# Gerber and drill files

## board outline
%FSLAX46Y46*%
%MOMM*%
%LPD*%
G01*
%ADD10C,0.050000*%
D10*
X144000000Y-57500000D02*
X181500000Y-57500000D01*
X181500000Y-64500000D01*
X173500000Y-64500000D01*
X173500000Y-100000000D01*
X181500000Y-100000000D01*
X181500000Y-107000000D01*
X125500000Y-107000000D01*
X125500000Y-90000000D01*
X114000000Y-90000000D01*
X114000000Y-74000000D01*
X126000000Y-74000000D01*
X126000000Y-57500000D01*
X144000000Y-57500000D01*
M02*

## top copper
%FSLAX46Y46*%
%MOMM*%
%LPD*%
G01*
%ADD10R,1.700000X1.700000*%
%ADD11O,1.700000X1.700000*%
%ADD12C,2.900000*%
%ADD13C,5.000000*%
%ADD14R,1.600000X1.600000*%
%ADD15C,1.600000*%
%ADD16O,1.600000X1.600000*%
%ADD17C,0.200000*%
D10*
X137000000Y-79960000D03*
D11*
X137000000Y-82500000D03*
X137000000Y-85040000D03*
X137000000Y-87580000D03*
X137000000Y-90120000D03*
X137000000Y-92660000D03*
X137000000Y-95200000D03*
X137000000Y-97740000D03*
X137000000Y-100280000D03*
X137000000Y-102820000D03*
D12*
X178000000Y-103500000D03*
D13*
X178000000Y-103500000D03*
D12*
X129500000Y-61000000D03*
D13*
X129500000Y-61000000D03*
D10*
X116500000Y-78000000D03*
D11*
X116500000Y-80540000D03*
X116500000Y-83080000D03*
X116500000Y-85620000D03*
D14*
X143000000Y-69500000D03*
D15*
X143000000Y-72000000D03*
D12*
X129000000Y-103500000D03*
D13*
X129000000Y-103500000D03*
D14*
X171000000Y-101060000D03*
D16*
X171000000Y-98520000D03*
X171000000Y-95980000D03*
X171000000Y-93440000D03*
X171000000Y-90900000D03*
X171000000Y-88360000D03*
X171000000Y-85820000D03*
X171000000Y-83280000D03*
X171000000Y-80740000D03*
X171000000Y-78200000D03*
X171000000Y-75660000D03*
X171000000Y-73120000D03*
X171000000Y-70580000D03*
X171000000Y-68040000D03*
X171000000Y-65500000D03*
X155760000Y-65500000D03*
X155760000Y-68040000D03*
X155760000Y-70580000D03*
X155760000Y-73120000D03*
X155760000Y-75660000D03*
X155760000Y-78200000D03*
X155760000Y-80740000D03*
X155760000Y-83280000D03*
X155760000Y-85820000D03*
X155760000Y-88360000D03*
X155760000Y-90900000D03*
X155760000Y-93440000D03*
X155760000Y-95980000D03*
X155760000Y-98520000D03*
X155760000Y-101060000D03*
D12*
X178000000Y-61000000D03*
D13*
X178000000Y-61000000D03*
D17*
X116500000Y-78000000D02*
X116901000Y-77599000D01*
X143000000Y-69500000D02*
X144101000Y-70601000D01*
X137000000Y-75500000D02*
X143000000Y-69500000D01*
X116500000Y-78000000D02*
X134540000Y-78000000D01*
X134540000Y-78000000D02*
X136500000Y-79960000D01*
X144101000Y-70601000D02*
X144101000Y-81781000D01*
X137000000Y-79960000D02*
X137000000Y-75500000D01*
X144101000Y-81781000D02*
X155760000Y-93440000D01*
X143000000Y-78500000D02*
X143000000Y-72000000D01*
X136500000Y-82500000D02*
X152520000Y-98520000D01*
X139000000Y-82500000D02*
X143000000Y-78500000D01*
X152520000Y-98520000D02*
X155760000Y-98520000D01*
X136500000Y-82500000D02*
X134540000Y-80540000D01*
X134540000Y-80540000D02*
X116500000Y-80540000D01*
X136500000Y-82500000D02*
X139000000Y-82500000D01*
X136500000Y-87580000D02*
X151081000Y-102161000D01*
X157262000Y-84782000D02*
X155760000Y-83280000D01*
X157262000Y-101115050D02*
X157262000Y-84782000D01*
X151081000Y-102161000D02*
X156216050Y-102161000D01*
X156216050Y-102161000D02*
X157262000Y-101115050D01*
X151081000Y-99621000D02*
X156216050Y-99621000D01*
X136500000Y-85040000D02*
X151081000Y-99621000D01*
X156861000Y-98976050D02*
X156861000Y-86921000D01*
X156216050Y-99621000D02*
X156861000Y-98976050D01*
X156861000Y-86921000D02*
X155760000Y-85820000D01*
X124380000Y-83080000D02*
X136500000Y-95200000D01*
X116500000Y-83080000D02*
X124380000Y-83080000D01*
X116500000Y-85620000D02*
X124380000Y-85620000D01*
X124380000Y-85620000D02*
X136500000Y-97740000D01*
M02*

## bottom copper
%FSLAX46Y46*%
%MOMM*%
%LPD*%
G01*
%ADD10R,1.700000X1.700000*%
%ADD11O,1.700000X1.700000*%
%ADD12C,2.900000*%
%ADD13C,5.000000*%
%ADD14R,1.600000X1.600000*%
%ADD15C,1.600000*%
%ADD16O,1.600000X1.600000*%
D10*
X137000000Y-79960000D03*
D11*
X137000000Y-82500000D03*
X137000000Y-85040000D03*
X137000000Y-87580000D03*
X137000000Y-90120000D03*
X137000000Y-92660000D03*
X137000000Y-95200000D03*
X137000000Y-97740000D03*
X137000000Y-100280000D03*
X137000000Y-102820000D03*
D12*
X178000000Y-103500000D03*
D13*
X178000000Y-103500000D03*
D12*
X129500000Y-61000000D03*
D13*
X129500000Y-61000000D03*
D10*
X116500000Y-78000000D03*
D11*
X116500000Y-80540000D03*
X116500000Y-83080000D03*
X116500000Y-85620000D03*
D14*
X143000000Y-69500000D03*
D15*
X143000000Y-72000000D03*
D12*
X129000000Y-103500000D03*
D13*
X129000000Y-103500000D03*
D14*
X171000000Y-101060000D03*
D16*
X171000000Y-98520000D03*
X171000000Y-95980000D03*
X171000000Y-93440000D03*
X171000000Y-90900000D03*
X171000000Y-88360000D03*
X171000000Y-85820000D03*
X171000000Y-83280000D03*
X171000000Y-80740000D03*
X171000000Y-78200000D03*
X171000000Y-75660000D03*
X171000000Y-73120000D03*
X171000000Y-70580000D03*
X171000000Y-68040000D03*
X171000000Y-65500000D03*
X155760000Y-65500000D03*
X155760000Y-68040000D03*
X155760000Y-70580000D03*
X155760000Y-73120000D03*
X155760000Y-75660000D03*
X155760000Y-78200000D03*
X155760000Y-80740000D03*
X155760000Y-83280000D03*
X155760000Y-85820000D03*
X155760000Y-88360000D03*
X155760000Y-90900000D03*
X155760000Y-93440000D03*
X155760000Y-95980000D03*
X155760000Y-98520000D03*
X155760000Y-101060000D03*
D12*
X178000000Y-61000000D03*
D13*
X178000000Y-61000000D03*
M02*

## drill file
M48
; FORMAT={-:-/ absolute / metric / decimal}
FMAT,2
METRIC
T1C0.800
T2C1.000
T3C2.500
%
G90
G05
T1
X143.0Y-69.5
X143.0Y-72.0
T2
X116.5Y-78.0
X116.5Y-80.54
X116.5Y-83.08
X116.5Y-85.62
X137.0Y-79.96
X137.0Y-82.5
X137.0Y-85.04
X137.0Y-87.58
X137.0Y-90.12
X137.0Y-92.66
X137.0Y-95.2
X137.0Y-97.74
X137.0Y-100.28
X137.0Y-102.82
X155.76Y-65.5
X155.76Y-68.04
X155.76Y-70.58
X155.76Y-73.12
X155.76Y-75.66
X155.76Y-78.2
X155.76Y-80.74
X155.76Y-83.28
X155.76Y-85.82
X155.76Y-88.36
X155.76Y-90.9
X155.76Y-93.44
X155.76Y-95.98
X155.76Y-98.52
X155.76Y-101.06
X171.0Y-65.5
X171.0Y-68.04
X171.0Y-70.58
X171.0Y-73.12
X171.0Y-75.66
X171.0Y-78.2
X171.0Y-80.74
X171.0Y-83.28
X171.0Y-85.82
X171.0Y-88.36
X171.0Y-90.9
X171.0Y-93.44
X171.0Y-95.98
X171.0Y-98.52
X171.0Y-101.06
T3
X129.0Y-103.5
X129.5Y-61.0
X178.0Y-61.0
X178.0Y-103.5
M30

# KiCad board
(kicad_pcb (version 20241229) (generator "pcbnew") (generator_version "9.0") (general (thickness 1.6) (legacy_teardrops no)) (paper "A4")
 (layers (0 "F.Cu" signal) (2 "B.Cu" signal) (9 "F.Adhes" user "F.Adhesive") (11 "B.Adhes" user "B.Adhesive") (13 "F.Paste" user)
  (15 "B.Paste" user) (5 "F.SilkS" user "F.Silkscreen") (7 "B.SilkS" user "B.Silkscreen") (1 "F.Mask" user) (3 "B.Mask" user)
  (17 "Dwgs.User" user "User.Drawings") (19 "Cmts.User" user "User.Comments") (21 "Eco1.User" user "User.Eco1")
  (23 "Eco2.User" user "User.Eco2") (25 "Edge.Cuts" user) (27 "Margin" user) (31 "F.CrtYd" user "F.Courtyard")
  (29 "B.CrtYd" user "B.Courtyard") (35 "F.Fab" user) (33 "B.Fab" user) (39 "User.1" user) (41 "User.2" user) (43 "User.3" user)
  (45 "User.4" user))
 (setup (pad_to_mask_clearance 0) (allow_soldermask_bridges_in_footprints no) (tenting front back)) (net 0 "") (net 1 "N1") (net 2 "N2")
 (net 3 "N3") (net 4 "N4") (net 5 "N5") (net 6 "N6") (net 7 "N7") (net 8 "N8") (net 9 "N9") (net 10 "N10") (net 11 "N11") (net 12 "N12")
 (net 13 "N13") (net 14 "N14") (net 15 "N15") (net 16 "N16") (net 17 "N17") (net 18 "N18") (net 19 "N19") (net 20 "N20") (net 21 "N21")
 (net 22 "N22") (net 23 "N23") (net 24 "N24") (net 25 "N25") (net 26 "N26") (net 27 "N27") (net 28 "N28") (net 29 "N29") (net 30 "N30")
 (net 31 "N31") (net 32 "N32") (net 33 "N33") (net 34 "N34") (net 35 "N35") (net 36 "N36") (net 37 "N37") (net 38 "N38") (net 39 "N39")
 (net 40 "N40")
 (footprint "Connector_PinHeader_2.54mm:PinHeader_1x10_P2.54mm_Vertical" (layer "F.Cu") (at 137 79.96)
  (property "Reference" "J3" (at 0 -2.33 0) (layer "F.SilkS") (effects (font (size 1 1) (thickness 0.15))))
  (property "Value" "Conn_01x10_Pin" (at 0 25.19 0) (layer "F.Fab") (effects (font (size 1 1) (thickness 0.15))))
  (pad "1" thru_hole rect (at 0 0) (size 1.7 1.7) (drill 1) (layers "*.Cu" "*.Mask") (remove_unused_layers no) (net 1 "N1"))
  (pad "2" thru_hole oval (at 0 2.54) (size 1.7 1.7) (drill 1) (layers "*.Cu" "*.Mask") (remove_unused_layers no) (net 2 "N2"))
  (pad "3" thru_hole oval (at 0 5.08) (size 1.7 1.7) (drill 1) (layers "*.Cu" "*.Mask") (remove_unused_layers no) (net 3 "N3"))
  (pad "4" thru_hole oval (at 0 7.62) (size 1.7 1.7) (drill 1) (layers "*.Cu" "*.Mask") (remove_unused_layers no) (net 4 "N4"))
  (pad "5" thru_hole oval (at 0 10.16) (size 1.7 1.7) (drill 1) (layers "*.Cu" "*.Mask") (remove_unused_layers no) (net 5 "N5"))
  (pad "6" thru_hole oval (at 0 12.7) (size 1.7 1.7) (drill 1) (layers "*.Cu" "*.Mask") (remove_unused_layers no) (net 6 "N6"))
  (pad "7" thru_hole oval (at 0 15.24) (size 1.7 1.7) (drill 1) (layers "*.Cu" "*.Mask") (remove_unused_layers no) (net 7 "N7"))
  (pad "8" thru_hole oval (at 0 17.78) (size 1.7 1.7) (drill 1) (layers "*.Cu" "*.Mask") (remove_unused_layers no) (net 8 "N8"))
  (pad "9" thru_hole oval (at 0 20.32) (size 1.7 1.7) (drill 1) (layers "*.Cu" "*.Mask") (remove_unused_layers no) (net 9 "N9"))
  (pad "10" thru_hole oval (at 0 22.86) (size 1.7 1.7) (drill 1) (layers "*.Cu" "*.Mask") (remove_unused_layers no) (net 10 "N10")))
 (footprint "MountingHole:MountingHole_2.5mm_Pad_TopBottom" (layer "F.Cu") (at 178 103.5)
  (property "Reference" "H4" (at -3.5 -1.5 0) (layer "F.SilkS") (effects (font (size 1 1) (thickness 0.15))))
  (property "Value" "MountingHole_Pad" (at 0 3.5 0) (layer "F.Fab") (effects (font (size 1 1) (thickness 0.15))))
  (pad "1" thru_hole circle (at 0 0) (size 2.9 2.9) (drill 2.5) (layers "*.Cu" "*.Mask") (remove_unused_layers no) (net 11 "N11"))
  (pad "1" connect circle (at 0 0) (size 5 5) (layers "F.Cu" "F.Mask") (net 11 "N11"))
  (pad "1" connect circle (at 0 0) (size 5 5) (layers "B.Cu" "B.Mask") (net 11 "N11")))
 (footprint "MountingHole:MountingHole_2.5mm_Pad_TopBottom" (layer "F.Cu") (at 129.5 61)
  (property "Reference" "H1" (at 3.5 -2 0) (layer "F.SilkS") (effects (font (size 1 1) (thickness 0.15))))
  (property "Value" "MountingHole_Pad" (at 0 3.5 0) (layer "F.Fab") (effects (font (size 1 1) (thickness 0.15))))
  (pad "1" thru_hole circle (at 0 0) (size 2.9 2.9) (drill 2.5) (layers "*.Cu" "*.Mask") (remove_unused_layers no) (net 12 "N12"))
  (pad "1" connect circle (at 0 0) (size 5 5) (layers "F.Cu" "F.Mask") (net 12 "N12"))
  (pad "1" connect circle (at 0 0) (size 5 5) (layers "B.Cu" "B.Mask") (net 12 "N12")))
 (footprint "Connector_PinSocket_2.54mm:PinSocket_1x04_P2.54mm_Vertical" (layer "F.Cu") (at 116.5 78)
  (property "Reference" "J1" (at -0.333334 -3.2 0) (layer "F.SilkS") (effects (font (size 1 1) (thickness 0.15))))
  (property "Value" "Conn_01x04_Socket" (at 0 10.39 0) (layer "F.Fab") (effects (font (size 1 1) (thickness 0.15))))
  (pad "1" thru_hole rect (at 0 0) (size 1.7 1.7) (drill 1) (layers "*.Cu" "*.Mask") (remove_unused_layers no) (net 1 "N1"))
  (pad "2" thru_hole oval (at 0 2.54) (size 1.7 1.7) (drill 1) (layers "*.Cu" "*.Mask") (remove_unused_layers no) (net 2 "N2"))
  (pad "3" thru_hole oval (at 0 5.08) (size 1.7 1.7) (drill 1) (layers "*.Cu" "*.Mask") (remove_unused_layers no) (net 7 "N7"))
  (pad "4" thru_hole oval (at 0 7.62) (size 1.7 1.7) (drill 1) (layers "*.Cu" "*.Mask") (remove_unused_layers no) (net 8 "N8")))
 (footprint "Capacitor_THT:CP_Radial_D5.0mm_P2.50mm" (layer "F.Cu") (at 143 69.5 -90)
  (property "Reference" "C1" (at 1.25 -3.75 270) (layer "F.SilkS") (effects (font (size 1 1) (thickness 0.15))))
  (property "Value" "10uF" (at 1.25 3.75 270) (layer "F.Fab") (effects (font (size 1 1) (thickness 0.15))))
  (pad "1" thru_hole rect (at 0 0 270) (size 1.6 1.6) (drill 0.8) (layers "*.Cu" "*.Mask") (remove_unused_layers no) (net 1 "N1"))
  (pad "2" thru_hole circle (at 2.5 0 270) (size 1.6 1.6) (drill 0.8) (layers "*.Cu" "*.Mask") (remove_unused_layers no) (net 2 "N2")))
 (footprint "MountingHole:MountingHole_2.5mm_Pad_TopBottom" (layer "F.Cu") (at 129 103.5)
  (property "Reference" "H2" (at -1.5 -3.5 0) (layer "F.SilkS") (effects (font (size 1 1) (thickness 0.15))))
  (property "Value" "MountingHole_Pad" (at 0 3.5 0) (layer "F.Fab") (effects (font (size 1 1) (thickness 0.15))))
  (pad "1" thru_hole circle (at 0 0) (size 2.9 2.9) (drill 2.5) (layers "*.Cu" "*.Mask") (remove_unused_layers no) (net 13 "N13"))
  (pad "1" connect circle (at 0 0) (size 5 5) (layers "F.Cu" "F.Mask") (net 13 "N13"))
  (pad "1" connect circle (at 0 0) (size 5 5) (layers "B.Cu" "B.Mask") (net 13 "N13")))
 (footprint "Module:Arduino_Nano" (layer "F.Cu") (at 171 101.06 180)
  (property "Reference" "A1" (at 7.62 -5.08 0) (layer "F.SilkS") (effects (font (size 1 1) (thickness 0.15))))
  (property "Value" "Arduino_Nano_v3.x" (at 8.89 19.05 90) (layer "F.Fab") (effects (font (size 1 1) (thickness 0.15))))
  (pad "1" thru_hole rect (at 0 0 180) (size 1.6 1.6) (drill 1) (layers "*.Cu" "*.Mask") (remove_unused_layers no) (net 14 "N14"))
  (pad "2" thru_hole oval (at 0 2.54 180) (size 1.6 1.6) (drill 1) (layers "*.Cu" "*.Mask") (remove_unused_layers no) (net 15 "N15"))
  (pad "3" thru_hole oval (at 0 5.08 180) (size 1.6 1.6) (drill 1) (layers "*.Cu" "*.Mask") (remove_unused_layers no) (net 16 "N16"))
  (pad "4" thru_hole oval (at 0 7.62 180) (size 1.6 1.6) (drill 1) (layers "*.Cu" "*.Mask") (remove_unused_layers no) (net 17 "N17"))
  (pad "5" thru_hole oval (at 0 10.16 180) (size 1.6 1.6) (drill 1) (layers "*.Cu" "*.Mask") (remove_unused_layers no) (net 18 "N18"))
  (pad "6" thru_hole oval (at 0 12.7 180) (size 1.6 1.6) (drill 1) (layers "*.Cu" "*.Mask") (remove_unused_layers no) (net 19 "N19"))
  (pad "7" thru_hole oval (at 0 15.24 180) (size 1.6 1.6) (drill 1) (layers "*.Cu" "*.Mask") (remove_unused_layers no) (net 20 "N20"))
  (pad "8" thru_hole oval (at 0 17.78 180) (size 1.6 1.6) (drill 1) (layers "*.Cu" "*.Mask") (remove_unused_layers no) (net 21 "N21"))
  (pad "9" thru_hole oval (at 0 20.32 180) (size 1.6 1.6) (drill 1) (layers "*.Cu" "*.Mask") (remove_unused_layers no) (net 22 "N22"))
  (pad "10" thru_hole oval (at 0 22.86 180) (size 1.6 1.6) (drill 1) (layers "*.Cu" "*.Mask") (remove_unused_layers no) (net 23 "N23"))
  (pad "11" thru_hole oval (at 0 25.4 180) (size 1.6 1.6) (drill 1) (layers "*.Cu" "*.Mask") (remove_unused_layers no) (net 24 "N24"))
  (pad "12" thru_hole oval (at 0 27.94 180) (size 1.6 1.6) (drill 1) (layers "*.Cu" "*.Mask") (remove_unused_layers no) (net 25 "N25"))
  (pad "13" thru_hole oval (at 0 30.48 180) (size 1.6 1.6) (drill 1) (layers "*.Cu" "*.Mask") (remove_unused_layers no) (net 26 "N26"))
  (pad "14" thru_hole oval (at 0 33.02 180) (size 1.6 1.6) (drill 1) (layers "*.Cu" "*.Mask") (remove_unused_layers no) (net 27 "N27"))
  (pad "15" thru_hole oval (at 0 35.56 180) (size 1.6 1.6) (drill 1) (layers "*.Cu" "*.Mask") (remove_unused_layers no) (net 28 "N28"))
  (pad "16" thru_hole oval (at 15.24 35.56 180) (size 1.6 1.6) (drill 1) (layers "*.Cu" "*.Mask") (remove_unused_layers no) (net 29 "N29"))
  (pad "17" thru_hole oval (at 15.24 33.02 180) (size 1.6 1.6) (drill 1) (layers "*.Cu" "*.Mask") (remove_unused_layers no) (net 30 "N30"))
  (pad "18" thru_hole oval (at 15.24 30.48 180) (size 1.6 1.6) (drill 1) (layers "*.Cu" "*.Mask") (remove_unused_layers no) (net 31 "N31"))
  (pad "19" thru_hole oval (at 15.24 27.94 180) (size 1.6 1.6) (drill 1) (layers "*.Cu" "*.Mask") (remove_unused_layers no) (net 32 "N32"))
  (pad "20" thru_hole oval (at 15.24 25.4 180) (size 1.6 1.6) (drill 1) (layers "*.Cu" "*.Mask") (remove_unused_layers no) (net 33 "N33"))
  (pad "21" thru_hole oval (at 15.24 22.86 180) (size 1.6 1.6) (drill 1) (layers "*.Cu" "*.Mask") (remove_unused_layers no) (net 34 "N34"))
  (pad "22" thru_hole oval (at 15.24 20.32 180) (size 1.6 1.6) (drill 1) (layers "*.Cu" "*.Mask") (remove_unused_layers no) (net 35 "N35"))
  (pad "23" thru_hole oval (at 15.24 17.78 180) (size 1.6 1.6) (drill 1) (layers "*.Cu" "*.Mask") (remove_unused_layers no) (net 4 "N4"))
  (pad "24" thru_hole oval (at 15.24 15.24 180) (size 1.6 1.6) (drill 1) (layers "*.Cu" "*.Mask") (remove_unused_layers no) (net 3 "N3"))
  (pad "25" thru_hole oval (at 15.24 12.7 180) (size 1.6 1.6) (drill 1) (layers "*.Cu" "*.Mask") (remove_unused_layers no) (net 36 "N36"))
  (pad "26" thru_hole oval (at 15.24 10.16 180) (size 1.6 1.6) (drill 1) (layers "*.Cu" "*.Mask") (remove_unused_layers no) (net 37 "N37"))
  (pad "27" thru_hole oval (at 15.24 7.62 180) (size 1.6 1.6) (drill 1) (layers "*.Cu" "*.Mask") (remove_unused_layers no) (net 1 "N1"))
  (pad "28" thru_hole oval (at 15.24 5.08 180) (size 1.6 1.6) (drill 1) (layers "*.Cu" "*.Mask") (remove_unused_layers no) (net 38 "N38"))
  (pad "29" thru_hole oval (at 15.24 2.54 180) (size 1.6 1.6) (drill 1) (layers "*.Cu" "*.Mask") (remove_unused_layers no) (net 2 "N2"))
  (pad "30" thru_hole oval (at 15.24 0 180) (size 1.6 1.6) (drill 1) (layers "*.Cu" "*.Mask") (remove_unused_layers no) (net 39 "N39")))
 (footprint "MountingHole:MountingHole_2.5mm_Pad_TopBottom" (layer "F.Cu") (at 178 61)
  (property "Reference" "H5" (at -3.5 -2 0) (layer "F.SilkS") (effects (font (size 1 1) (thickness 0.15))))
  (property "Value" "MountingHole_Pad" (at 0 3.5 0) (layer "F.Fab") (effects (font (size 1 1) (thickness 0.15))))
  (pad "1" thru_hole circle (at 0 0) (size 2.9 2.9) (drill 2.5) (layers "*.Cu" "*.Mask") (remove_unused_layers no) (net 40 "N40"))
  (pad "1" connect circle (at 0 0) (size 5 5) (layers "F.Cu" "F.Mask") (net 40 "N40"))
  (pad "1" connect circle (at 0 0) (size 5 5) (layers "B.Cu" "B.Mask") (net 40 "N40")))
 (gr_poly
  (pts (xy 144 57.5) (xy 181.5 57.5) (xy 181.5 64.5) (xy 173.5 64.5) (xy 173.5 100) (xy 181.5 100) (xy 181.5 107) (xy 125.5 107)
   (xy 125.5 90) (xy 114 90) (xy 114 74) (xy 126 74) (xy 126 57.5))
  (stroke (width 0.05) (type solid)) (fill no) (layer "Edge.Cuts"))
 (segment (start 116.5 78) (end 116.901 77.599) (width 0.2) (layer "F.Cu") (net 1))
 (segment (start 143 69.5) (end 144.101 70.601) (width 0.2) (layer "F.Cu") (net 1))
 (segment (start 137 75.5) (end 143 69.5) (width 0.2) (layer "F.Cu") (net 1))
 (segment (start 116.5 78) (end 134.54 78) (width 0.2) (layer "F.Cu") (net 1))
 (segment (start 134.54 78) (end 136.5 79.96) (width 0.2) (layer "F.Cu") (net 1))
 (segment (start 144.101 70.601) (end 144.101 81.781) (width 0.2) (layer "F.Cu") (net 1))
 (segment (start 137 79.96) (end 137 75.5) (width 0.2) (layer "F.Cu") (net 1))
 (segment (start 144.101 81.781) (end 155.76 93.44) (width 0.2) (layer "F.Cu") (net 1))
 (segment (start 143 78.5) (end 143 72) (width 0.2) (layer "F.Cu") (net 2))
 (segment (start 136.5 82.5) (end 152.52 98.52) (width 0.2) (layer "F.Cu") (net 2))
 (segment (start 139 82.5) (end 143 78.5) (width 0.2) (layer "F.Cu") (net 2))
 (segment (start 152.52 98.52) (end 155.76 98.52) (width 0.2) (layer "F.Cu") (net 2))
 (segment (start 136.5 82.5) (end 134.54 80.54) (width 0.2) (layer "F.Cu") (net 2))
 (segment (start 134.54 80.54) (end 116.5 80.54) (width 0.2) (layer "F.Cu") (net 2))
 (segment (start 136.5 82.5) (end 139 82.5) (width 0.2) (layer "F.Cu") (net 2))
 (segment (start 136.5 87.58) (end 151.081 102.161) (width 0.2) (layer "F.Cu") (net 4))
 (segment (start 157.262 84.782) (end 155.76 83.28) (width 0.2) (layer "F.Cu") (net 4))
 (segment (start 157.262 101.11505) (end 157.262 84.782) (width 0.2) (layer "F.Cu") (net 4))
 (segment (start 151.081 102.161) (end 156.21605 102.161) (width 0.2) (layer "F.Cu") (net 4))
 (segment (start 156.21605 102.161) (end 157.262 101.11505) (width 0.2) (layer "F.Cu") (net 4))
 (segment (start 151.081 99.621) (end 156.21605 99.621) (width 0.2) (layer "F.Cu") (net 3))
 (segment (start 136.5 85.04) (end 151.081 99.621) (width 0.2) (layer "F.Cu") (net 3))
 (segment (start 156.861 98.97605) (end 156.861 86.921) (width 0.2) (layer "F.Cu") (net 3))
 (segment (start 156.21605 99.621) (end 156.861 98.97605) (width 0.2) (layer "F.Cu") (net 3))
 (segment (start 156.861 86.921) (end 155.76 85.82) (width 0.2) (layer "F.Cu") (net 3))
 (segment (start 124.38 83.08) (end 136.5 95.2) (width 0.2) (layer "F.Cu") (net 7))
 (segment (start 116.5 83.08) (end 124.38 83.08) (width 0.2) (layer "F.Cu") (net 7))
 (segment (start 116.5 85.62) (end 124.38 85.62) (width 0.2) (layer "F.Cu") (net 8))
 (segment (start 124.38 85.62) (end 136.5 97.74) (width 0.2) (layer "F.Cu") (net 8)))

